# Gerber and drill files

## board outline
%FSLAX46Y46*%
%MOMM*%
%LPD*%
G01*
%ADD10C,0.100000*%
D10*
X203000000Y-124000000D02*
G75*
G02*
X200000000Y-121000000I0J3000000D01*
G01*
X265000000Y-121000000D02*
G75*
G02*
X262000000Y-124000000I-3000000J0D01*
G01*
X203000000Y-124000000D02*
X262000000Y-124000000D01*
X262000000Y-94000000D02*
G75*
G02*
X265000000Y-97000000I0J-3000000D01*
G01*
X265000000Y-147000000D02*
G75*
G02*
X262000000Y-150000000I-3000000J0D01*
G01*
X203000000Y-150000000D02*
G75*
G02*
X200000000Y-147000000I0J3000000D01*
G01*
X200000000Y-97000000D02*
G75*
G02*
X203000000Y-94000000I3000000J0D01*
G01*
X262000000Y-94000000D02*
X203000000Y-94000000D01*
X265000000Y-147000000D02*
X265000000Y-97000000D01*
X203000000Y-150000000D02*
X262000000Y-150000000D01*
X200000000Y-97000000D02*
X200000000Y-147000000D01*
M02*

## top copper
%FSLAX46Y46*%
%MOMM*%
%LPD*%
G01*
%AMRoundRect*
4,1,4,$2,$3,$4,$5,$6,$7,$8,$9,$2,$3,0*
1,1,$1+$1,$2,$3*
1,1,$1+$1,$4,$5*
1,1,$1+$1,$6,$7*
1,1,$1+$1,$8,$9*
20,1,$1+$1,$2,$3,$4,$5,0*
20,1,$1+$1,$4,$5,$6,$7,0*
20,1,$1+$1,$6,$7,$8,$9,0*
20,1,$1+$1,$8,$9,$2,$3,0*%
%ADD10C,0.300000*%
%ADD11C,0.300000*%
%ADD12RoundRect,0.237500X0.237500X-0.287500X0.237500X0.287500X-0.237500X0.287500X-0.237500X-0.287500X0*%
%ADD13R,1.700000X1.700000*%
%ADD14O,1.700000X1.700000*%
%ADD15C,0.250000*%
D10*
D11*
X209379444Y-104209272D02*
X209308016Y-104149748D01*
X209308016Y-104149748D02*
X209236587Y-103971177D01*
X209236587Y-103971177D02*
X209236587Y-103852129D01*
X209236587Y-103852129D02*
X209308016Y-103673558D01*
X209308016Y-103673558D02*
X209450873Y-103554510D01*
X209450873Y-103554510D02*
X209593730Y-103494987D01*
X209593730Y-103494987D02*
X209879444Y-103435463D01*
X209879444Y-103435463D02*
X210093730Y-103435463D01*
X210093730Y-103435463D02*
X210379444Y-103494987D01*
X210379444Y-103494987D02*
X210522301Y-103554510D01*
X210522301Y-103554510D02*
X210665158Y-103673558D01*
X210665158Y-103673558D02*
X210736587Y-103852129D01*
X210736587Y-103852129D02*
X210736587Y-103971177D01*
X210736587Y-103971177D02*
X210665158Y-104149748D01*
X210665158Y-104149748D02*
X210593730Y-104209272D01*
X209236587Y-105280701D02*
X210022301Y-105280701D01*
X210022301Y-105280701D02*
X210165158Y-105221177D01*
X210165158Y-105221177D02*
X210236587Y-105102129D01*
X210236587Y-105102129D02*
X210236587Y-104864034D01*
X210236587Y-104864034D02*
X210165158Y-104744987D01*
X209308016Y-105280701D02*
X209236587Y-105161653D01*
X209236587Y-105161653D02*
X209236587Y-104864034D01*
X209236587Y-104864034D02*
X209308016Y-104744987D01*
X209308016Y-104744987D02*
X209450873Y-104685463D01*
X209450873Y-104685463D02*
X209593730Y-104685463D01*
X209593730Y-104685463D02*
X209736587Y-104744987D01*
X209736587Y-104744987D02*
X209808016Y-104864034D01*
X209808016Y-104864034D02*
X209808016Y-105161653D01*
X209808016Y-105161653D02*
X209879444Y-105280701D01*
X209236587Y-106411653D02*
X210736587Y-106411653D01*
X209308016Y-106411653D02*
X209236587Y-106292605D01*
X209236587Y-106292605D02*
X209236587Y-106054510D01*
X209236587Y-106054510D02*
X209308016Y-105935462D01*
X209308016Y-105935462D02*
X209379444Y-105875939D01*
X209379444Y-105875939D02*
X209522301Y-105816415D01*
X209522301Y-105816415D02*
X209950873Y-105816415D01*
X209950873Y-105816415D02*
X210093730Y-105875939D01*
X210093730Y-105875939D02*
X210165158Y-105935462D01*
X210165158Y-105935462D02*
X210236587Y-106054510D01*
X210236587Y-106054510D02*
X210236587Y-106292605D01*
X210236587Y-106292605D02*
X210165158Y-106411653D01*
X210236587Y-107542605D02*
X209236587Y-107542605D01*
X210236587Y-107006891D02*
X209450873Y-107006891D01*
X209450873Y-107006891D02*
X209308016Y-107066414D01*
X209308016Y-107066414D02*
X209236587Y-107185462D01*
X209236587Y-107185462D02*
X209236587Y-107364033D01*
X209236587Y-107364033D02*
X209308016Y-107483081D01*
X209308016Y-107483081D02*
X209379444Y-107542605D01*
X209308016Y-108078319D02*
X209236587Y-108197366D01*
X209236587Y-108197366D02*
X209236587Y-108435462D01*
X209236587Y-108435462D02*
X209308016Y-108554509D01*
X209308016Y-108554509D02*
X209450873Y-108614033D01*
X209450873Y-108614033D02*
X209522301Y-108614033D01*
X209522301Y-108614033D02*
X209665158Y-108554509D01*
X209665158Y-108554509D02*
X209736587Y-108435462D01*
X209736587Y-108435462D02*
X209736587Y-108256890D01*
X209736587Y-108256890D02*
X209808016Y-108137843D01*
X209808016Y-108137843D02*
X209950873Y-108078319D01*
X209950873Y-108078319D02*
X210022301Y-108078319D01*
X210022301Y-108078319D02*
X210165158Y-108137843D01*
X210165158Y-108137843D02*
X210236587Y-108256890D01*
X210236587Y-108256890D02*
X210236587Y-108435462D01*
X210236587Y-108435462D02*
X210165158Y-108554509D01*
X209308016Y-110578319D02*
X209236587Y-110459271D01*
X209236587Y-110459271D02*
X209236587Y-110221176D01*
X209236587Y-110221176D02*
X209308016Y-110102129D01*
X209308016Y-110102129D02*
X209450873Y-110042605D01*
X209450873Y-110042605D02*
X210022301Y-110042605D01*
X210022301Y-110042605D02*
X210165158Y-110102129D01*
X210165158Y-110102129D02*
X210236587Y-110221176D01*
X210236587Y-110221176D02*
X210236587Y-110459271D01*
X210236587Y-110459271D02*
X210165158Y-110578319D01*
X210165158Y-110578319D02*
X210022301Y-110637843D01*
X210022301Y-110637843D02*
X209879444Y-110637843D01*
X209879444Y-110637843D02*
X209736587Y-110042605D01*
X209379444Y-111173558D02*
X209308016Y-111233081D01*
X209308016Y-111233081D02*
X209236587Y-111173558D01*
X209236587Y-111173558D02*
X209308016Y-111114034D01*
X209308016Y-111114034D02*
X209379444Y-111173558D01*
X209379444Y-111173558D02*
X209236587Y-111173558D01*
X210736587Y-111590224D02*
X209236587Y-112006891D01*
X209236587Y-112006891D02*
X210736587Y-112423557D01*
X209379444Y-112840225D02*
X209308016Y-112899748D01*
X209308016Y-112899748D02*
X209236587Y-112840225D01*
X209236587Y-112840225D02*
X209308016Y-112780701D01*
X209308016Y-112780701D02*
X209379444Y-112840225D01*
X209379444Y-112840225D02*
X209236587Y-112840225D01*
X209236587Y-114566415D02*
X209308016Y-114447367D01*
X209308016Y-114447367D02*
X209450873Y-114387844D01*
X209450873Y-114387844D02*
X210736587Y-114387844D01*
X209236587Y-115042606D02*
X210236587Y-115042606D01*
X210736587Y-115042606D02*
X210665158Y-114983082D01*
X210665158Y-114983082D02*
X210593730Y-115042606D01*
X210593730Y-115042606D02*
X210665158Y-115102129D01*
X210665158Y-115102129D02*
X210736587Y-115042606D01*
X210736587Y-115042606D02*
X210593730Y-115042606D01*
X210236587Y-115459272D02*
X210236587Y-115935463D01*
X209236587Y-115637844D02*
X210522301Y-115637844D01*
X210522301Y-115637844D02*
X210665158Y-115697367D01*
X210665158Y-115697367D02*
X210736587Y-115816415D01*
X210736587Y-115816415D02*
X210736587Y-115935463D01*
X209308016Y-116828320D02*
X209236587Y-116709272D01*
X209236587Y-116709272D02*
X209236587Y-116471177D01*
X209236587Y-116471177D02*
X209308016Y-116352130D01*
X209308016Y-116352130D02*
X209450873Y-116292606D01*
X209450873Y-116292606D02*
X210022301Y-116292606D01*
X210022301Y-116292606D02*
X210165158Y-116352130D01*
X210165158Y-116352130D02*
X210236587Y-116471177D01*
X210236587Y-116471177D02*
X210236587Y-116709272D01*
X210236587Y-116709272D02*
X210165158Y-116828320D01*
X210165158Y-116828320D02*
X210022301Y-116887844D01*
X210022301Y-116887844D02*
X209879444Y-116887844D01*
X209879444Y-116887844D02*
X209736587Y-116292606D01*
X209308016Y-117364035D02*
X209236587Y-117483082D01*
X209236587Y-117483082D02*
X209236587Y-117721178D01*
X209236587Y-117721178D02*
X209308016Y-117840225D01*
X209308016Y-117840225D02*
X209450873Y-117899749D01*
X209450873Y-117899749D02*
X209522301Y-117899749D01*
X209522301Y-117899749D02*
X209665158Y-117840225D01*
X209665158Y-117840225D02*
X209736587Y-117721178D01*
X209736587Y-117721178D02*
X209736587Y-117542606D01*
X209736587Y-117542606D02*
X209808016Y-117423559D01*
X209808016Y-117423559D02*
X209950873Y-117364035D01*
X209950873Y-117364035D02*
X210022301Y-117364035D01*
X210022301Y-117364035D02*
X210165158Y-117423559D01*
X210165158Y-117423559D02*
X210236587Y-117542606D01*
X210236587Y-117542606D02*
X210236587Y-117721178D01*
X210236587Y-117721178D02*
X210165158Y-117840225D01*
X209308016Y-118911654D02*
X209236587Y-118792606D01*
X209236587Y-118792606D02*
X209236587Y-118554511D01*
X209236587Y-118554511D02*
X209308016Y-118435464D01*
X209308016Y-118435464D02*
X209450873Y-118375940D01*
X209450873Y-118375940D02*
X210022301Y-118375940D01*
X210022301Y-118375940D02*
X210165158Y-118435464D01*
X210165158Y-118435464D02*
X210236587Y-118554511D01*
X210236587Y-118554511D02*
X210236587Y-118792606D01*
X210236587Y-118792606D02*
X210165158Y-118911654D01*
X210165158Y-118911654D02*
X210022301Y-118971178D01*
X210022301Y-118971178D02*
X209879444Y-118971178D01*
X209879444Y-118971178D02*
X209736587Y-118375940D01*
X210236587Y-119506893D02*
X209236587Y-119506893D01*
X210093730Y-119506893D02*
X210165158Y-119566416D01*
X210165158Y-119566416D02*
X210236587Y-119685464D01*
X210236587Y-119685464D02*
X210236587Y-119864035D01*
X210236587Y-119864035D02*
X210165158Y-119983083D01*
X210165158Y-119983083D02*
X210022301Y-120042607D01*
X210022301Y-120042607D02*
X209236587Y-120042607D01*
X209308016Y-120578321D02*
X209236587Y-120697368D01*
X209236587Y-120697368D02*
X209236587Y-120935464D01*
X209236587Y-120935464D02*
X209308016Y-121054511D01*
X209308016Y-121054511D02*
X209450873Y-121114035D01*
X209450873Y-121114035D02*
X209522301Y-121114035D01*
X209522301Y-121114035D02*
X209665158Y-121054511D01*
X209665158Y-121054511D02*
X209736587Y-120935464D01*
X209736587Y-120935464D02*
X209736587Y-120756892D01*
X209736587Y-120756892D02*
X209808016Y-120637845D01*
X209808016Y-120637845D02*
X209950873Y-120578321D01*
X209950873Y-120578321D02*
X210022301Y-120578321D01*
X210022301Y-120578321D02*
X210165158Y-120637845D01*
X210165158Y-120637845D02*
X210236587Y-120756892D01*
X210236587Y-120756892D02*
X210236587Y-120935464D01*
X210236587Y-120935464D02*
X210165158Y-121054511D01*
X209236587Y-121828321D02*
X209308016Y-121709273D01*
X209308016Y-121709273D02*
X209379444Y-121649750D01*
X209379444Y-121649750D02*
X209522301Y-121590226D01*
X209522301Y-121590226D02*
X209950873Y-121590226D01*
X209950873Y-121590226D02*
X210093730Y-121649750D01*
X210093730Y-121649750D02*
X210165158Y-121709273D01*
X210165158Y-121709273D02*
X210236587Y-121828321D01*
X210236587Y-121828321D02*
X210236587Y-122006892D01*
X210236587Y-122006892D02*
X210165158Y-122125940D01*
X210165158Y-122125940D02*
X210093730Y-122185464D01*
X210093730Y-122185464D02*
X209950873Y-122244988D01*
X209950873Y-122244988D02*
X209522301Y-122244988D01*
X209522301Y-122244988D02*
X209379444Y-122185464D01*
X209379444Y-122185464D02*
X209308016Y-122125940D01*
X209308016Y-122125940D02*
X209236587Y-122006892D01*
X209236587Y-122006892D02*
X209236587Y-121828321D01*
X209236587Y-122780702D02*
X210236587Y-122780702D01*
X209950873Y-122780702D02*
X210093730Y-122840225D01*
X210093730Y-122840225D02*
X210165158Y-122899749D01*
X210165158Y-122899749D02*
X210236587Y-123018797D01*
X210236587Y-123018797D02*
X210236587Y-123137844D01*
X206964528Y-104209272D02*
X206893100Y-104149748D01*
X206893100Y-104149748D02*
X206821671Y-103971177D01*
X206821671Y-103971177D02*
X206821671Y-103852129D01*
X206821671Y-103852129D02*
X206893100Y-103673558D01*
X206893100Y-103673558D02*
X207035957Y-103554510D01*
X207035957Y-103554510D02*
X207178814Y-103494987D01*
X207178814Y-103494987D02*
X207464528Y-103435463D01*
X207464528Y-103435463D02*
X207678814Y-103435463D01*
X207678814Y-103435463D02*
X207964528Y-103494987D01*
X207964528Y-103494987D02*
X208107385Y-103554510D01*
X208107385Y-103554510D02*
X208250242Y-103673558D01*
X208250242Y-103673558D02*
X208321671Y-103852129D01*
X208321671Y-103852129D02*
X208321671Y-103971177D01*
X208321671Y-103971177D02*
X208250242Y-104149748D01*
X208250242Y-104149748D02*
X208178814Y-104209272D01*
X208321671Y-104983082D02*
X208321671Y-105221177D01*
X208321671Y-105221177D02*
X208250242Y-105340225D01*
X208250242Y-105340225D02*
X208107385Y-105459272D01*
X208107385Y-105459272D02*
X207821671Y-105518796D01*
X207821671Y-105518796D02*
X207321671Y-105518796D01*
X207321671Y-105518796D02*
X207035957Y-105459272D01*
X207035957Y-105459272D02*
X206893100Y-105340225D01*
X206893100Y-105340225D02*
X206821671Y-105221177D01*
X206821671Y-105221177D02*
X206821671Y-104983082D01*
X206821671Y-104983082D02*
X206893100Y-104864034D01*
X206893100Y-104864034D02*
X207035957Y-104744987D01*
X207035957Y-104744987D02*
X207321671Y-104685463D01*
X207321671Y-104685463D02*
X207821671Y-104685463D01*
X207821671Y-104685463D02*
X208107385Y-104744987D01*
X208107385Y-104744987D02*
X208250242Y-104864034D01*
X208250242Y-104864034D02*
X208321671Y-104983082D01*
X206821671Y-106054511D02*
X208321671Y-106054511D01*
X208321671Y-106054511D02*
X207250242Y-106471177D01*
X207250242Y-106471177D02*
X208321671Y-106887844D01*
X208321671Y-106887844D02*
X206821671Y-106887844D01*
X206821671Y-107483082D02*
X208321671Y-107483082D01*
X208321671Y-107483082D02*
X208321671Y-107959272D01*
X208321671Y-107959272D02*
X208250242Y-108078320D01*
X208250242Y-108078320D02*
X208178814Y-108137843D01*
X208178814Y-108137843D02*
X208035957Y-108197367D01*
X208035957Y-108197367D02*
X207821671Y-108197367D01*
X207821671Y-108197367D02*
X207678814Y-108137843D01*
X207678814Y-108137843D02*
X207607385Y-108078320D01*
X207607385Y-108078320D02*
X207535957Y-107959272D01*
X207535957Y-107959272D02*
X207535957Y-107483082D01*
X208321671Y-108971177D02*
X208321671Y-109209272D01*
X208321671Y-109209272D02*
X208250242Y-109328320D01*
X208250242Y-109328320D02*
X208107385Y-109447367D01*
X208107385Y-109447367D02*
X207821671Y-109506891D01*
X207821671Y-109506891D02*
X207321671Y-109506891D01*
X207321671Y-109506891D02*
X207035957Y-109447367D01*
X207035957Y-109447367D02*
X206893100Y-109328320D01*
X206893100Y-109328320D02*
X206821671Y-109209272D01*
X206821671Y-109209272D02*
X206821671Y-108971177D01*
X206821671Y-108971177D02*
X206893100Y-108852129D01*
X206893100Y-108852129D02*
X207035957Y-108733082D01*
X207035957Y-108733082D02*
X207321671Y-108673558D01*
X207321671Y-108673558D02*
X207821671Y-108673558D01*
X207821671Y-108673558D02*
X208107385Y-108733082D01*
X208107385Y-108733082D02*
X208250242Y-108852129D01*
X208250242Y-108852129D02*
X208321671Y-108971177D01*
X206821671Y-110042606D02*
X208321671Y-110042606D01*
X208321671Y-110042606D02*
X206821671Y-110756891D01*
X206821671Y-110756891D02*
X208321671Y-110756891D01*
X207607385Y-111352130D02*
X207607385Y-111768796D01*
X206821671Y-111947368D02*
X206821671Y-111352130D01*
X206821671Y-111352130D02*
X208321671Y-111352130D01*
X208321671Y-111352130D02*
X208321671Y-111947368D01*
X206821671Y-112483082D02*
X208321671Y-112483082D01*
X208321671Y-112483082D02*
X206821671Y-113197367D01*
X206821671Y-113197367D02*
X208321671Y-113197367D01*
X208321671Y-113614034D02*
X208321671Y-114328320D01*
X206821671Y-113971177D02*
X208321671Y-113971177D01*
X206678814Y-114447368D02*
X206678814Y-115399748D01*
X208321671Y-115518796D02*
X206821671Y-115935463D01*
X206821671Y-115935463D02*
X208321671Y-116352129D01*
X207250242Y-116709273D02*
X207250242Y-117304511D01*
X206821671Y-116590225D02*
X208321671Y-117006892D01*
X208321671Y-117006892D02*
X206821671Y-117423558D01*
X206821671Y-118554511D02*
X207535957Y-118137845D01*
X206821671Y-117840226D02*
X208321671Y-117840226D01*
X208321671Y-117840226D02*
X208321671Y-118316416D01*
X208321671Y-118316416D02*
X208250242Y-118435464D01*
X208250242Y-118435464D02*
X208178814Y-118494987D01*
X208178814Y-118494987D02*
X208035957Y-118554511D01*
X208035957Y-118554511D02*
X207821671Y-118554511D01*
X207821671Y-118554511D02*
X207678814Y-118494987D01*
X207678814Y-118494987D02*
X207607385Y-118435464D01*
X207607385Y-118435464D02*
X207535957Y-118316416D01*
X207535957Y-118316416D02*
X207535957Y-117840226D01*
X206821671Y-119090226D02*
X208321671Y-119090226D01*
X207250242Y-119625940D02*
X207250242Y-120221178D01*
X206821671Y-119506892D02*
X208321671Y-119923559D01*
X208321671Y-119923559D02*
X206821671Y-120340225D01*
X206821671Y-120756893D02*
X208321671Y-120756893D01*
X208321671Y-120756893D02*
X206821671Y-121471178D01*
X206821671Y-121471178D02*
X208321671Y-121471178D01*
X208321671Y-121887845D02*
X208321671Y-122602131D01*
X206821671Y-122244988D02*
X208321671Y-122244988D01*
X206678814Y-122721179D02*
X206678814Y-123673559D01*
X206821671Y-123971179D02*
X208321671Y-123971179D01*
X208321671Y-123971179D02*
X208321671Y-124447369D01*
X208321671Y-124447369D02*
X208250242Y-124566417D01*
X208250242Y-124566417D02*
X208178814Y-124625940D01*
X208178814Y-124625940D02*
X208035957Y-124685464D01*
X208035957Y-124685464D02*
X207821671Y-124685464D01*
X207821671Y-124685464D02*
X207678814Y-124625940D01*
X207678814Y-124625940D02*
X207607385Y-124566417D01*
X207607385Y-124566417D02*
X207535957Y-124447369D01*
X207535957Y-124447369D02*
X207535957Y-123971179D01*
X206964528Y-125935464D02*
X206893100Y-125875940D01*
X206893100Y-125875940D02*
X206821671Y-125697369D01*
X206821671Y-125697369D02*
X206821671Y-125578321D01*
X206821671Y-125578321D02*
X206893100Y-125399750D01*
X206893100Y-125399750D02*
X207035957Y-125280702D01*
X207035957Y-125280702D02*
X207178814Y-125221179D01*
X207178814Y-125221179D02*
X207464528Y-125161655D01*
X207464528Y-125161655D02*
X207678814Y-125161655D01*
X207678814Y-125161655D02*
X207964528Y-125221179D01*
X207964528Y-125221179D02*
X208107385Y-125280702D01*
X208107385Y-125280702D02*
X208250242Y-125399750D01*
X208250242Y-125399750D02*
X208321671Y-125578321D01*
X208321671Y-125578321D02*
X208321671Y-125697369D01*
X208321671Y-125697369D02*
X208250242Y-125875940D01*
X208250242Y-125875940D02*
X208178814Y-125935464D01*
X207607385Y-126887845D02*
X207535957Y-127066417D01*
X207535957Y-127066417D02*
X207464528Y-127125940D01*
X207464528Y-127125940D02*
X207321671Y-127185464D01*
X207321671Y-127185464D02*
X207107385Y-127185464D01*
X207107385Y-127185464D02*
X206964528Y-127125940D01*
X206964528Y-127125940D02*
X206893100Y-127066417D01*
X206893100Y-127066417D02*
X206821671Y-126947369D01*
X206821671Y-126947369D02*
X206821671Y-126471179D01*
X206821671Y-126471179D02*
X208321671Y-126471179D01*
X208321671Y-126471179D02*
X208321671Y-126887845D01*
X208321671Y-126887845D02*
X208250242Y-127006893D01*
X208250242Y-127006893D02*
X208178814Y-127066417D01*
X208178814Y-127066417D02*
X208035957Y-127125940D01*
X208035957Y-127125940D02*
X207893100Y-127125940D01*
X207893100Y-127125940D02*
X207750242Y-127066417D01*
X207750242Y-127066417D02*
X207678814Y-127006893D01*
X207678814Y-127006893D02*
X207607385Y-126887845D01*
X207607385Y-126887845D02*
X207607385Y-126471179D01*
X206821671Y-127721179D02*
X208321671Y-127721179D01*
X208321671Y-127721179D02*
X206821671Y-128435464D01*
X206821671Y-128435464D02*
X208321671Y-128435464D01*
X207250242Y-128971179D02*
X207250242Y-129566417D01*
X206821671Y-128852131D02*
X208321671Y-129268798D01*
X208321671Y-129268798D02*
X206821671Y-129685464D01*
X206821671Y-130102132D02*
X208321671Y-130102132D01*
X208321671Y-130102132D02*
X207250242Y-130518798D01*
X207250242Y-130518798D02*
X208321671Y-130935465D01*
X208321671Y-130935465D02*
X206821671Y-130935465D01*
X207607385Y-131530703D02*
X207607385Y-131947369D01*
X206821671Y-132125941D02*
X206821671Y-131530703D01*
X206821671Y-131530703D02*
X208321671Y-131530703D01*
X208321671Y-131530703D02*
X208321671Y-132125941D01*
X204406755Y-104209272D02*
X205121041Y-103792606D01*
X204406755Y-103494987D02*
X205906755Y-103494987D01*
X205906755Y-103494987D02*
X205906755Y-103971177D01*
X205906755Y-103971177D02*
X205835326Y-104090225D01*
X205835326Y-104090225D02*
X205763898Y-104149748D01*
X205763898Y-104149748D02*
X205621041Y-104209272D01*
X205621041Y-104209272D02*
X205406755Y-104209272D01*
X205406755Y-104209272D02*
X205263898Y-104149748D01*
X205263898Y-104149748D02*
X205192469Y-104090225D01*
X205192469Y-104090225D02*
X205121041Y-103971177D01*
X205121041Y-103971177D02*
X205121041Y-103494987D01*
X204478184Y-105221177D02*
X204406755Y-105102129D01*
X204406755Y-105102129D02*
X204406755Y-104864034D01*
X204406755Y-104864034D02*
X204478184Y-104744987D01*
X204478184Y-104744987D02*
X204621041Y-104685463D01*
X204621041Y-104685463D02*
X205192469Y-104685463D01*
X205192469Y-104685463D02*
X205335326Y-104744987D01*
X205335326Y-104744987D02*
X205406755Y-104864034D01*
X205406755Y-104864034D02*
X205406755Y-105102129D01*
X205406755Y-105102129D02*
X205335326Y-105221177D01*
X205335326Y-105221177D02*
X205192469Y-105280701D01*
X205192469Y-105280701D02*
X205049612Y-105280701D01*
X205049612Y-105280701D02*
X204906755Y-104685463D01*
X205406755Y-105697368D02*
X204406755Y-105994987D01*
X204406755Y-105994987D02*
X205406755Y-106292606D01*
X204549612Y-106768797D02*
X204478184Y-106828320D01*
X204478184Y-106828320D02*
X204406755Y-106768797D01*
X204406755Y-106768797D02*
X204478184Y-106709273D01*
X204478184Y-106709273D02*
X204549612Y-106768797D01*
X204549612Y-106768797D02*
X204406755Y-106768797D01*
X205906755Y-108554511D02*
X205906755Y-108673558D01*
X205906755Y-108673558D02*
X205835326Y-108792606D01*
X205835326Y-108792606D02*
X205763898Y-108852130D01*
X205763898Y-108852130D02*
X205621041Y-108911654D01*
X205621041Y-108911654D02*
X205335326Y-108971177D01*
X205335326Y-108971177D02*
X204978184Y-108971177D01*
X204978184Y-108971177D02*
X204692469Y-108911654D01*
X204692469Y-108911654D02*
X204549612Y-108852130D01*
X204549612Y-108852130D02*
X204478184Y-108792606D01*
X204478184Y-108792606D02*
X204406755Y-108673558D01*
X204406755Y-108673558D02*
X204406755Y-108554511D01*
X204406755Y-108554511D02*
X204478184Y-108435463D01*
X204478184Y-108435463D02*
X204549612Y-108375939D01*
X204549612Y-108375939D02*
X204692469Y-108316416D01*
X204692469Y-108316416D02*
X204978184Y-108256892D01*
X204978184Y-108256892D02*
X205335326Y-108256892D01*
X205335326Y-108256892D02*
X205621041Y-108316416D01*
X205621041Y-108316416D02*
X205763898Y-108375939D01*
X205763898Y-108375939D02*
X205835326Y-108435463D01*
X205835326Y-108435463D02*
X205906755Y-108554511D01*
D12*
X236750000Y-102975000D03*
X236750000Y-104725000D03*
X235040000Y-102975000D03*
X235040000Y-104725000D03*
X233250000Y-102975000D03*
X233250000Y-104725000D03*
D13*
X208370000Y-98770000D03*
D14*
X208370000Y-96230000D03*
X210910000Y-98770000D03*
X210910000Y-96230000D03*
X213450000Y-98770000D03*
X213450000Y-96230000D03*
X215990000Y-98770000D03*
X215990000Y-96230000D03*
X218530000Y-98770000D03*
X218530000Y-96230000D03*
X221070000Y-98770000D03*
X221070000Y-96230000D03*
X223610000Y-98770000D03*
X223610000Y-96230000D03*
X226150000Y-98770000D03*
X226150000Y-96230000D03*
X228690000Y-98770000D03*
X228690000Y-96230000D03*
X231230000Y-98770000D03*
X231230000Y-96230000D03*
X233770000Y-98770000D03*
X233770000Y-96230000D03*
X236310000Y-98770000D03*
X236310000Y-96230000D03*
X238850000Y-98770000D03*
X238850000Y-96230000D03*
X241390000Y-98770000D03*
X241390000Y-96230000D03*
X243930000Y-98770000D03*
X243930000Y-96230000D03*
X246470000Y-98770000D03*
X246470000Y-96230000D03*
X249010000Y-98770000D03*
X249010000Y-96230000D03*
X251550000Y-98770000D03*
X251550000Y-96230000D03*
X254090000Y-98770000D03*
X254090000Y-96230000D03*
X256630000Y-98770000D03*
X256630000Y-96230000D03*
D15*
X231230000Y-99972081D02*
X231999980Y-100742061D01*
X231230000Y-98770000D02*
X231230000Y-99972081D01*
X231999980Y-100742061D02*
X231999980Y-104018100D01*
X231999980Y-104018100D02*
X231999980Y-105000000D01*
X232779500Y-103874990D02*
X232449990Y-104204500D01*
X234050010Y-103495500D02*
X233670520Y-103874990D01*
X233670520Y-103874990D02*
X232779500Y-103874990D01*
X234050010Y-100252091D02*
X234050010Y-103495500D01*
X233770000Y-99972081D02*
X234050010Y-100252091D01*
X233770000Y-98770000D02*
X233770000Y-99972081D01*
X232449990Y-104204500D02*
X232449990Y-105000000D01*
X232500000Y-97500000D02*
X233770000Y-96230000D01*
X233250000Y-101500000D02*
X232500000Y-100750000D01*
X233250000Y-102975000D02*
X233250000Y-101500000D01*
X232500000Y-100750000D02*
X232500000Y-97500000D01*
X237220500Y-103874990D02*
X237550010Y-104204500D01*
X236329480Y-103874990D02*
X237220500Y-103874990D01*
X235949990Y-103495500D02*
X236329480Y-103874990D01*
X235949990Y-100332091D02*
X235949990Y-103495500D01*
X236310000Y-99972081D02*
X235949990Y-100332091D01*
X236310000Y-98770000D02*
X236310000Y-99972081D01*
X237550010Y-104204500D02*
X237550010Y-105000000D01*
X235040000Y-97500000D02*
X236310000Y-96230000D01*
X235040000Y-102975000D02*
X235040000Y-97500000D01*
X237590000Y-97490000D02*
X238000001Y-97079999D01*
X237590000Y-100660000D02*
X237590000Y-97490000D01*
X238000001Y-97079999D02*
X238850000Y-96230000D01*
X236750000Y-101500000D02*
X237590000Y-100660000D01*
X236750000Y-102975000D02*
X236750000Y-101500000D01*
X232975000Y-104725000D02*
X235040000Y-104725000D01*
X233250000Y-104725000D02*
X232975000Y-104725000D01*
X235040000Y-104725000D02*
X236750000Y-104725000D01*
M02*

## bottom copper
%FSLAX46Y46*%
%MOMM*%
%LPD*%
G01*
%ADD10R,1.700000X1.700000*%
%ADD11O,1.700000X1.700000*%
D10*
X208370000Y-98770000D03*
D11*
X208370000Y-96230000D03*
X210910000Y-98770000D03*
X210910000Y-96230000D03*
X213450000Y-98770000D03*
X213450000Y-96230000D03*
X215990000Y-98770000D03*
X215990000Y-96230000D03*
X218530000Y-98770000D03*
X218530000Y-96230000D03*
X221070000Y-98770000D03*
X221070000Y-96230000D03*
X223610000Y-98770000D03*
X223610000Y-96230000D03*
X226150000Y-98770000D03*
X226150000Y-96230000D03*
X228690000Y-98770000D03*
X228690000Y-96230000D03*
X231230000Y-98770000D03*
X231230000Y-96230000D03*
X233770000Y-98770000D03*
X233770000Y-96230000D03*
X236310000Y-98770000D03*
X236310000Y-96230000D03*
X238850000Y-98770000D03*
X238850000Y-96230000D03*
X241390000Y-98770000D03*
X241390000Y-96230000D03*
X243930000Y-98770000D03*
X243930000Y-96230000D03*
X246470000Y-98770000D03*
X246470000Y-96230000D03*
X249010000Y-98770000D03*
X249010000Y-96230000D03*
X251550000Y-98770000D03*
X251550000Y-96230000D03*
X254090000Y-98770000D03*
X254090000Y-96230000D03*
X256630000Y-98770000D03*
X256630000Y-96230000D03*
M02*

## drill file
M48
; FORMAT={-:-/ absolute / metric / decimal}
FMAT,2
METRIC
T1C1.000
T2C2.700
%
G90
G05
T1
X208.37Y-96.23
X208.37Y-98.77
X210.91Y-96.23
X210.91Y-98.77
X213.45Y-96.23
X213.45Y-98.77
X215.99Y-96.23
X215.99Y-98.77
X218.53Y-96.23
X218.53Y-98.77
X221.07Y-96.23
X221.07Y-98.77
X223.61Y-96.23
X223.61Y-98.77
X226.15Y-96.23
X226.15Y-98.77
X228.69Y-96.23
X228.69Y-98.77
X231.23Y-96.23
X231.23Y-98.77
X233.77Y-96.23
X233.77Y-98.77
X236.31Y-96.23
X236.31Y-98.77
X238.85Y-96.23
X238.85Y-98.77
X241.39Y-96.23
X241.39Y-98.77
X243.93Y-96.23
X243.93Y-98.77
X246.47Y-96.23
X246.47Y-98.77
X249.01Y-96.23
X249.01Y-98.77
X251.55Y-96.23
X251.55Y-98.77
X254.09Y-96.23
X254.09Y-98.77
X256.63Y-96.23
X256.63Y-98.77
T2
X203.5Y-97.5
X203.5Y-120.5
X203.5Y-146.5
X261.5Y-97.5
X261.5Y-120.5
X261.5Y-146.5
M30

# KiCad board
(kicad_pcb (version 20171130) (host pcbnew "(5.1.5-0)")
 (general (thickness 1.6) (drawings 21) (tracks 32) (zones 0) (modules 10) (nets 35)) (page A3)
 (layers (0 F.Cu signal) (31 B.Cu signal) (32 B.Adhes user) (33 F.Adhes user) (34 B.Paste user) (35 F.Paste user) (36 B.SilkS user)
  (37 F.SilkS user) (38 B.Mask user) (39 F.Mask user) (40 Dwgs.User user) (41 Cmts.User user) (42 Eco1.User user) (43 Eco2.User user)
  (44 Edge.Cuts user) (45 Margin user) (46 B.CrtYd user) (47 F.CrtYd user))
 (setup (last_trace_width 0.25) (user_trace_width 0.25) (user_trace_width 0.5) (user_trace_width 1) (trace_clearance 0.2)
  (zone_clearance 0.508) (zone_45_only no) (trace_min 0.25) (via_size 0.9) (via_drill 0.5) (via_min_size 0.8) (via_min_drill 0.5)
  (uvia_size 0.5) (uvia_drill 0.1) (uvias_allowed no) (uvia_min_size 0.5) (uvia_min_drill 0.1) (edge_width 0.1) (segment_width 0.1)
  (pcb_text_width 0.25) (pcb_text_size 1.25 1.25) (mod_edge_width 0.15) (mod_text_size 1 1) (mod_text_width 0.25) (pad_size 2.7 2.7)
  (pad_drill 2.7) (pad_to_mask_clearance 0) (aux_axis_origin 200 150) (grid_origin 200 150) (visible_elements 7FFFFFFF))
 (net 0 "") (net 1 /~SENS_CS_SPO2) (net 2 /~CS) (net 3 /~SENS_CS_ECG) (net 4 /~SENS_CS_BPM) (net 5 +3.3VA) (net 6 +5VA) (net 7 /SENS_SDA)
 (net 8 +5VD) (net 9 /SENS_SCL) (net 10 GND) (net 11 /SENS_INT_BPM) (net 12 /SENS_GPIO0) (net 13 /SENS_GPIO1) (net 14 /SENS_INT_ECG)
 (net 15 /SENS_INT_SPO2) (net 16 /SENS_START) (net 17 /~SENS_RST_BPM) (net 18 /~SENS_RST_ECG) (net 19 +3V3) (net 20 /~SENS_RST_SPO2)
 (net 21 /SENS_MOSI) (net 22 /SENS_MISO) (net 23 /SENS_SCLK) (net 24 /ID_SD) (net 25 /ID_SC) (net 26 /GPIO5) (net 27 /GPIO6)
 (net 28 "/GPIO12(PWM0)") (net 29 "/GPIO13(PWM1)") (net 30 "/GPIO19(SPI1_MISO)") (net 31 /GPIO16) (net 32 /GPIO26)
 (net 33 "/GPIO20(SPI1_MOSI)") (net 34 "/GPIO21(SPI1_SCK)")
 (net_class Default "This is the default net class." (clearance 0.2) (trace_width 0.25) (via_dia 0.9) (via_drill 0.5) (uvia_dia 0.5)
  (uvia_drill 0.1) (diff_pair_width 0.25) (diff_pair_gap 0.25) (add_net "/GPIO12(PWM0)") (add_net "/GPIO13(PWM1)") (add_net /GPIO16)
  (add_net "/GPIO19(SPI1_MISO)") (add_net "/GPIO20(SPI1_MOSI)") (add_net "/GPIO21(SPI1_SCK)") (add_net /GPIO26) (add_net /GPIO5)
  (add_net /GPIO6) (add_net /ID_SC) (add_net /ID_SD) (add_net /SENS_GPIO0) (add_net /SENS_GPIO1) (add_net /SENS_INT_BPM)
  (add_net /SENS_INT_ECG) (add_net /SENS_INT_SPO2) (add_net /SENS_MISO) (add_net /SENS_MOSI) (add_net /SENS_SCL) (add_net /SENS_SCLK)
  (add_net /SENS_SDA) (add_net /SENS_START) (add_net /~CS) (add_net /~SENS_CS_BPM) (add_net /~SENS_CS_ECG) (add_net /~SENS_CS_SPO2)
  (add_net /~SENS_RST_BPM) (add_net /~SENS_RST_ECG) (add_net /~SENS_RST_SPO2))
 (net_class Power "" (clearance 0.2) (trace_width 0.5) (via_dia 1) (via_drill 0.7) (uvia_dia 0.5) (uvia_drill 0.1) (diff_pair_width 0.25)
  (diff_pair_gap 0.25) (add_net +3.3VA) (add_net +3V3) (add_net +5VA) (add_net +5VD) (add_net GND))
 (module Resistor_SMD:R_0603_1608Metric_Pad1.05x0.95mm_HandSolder (layer F.Cu) (at 236.75 103.85 90)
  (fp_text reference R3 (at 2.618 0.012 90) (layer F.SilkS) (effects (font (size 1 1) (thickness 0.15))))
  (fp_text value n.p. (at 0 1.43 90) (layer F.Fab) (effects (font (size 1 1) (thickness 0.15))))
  (pad 2 smd roundrect (at 0.875 0 90) (size 1.05 0.95) (layers F.Cu F.Paste F.Mask) (roundrect_rratio 0.25) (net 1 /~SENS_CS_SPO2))
  (pad 1 smd roundrect (at -0.875 0 90) (size 1.05 0.95) (layers F.Cu F.Paste F.Mask) (roundrect_rratio 0.25) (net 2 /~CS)))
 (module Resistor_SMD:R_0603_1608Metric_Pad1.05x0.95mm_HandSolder (layer F.Cu) (at 235.04 103.85 90)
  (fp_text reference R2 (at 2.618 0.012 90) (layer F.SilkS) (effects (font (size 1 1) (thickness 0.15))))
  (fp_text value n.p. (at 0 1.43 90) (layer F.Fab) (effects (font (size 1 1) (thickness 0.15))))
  (pad 2 smd roundrect (at 0.875 0 90) (size 1.05 0.95) (layers F.Cu F.Paste F.Mask) (roundrect_rratio 0.25) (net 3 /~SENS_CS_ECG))
  (pad 1 smd roundrect (at -0.875 0 90) (size 1.05 0.95) (layers F.Cu F.Paste F.Mask) (roundrect_rratio 0.25) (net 2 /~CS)))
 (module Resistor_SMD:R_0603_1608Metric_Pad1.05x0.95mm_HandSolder (layer F.Cu) (at 233.25 103.85 90)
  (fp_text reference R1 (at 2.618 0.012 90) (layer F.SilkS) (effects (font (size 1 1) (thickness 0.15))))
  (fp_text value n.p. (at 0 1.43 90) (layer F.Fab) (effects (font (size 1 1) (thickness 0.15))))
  (pad 2 smd roundrect (at 0.875 0 90) (size 1.05 0.95) (layers F.Cu F.Paste F.Mask) (roundrect_rratio 0.25) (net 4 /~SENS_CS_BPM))
  (pad 1 smd roundrect (at -0.875 0 90) (size 1.05 0.95) (layers F.Cu F.Paste F.Mask) (roundrect_rratio 0.25) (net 2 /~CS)))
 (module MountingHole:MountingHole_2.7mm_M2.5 (layer F.Cu) (at 261.5 146.5)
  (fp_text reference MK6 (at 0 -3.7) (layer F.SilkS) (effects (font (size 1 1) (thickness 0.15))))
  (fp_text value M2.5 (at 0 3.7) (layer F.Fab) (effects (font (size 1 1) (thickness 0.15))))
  (pad 1 np_thru_hole circle (at 0 0) (size 2.7 2.7) (drill 2.7) (layers *.Cu *.Mask)))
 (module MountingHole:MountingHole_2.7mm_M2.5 (layer F.Cu) (at 203.5 146.5)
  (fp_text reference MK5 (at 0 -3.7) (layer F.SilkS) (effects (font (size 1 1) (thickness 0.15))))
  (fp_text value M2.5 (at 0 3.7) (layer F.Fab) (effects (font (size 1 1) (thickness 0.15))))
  (pad 1 np_thru_hole circle (at 0 0) (size 2.7 2.7) (drill 2.7) (layers *.Cu *.Mask)))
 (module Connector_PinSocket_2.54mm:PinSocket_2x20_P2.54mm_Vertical (layer B.Cu) (at 208.37 98.77 270)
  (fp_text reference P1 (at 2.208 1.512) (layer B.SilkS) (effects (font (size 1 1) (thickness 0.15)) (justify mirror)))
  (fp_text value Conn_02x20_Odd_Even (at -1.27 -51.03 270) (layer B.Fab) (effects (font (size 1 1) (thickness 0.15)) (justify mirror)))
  (pad 1 thru_hole rect (at 0 0 270) (size 1.7 1.7) (drill 1) (layers *.Cu *.Mask) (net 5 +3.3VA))
  (pad 2 thru_hole oval (at -2.54 0 270) (size 1.7 1.7) (drill 1) (layers *.Cu *.Mask) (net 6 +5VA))
  (pad 3 thru_hole oval (at 0 -2.54 270) (size 1.7 1.7) (drill 1) (layers *.Cu *.Mask) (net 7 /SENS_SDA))
  (pad 4 thru_hole oval (at -2.54 -2.54 270) (size 1.7 1.7) (drill 1) (layers *.Cu *.Mask) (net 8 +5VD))
  (pad 5 thru_hole oval (at 0 -5.08 270) (size 1.7 1.7) (drill 1) (layers *.Cu *.Mask) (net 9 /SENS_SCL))
  (pad 6 thru_hole oval (at -2.54 -5.08 270) (size 1.7 1.7) (drill 1) (layers *.Cu *.Mask) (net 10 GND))
  (pad 7 thru_hole oval (at 0 -7.62 270) (size 1.7 1.7) (drill 1) (layers *.Cu *.Mask) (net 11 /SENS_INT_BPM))
  (pad 8 thru_hole oval (at -2.54 -7.62 270) (size 1.7 1.7) (drill 1) (layers *.Cu *.Mask) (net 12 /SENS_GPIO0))
  (pad 9 thru_hole oval (at 0 -10.16 270) (size 1.7 1.7) (drill 1) (layers *.Cu *.Mask) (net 10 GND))
  (pad 10 thru_hole oval (at -2.54 -10.16 270) (size 1.7 1.7) (drill 1) (layers *.Cu *.Mask) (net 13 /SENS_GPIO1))
  (pad 11 thru_hole oval (at 0 -12.7 270) (size 1.7 1.7) (drill 1) (layers *.Cu *.Mask) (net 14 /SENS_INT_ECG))
  (pad 12 thru_hole oval (at -2.54 -12.7 270) (size 1.7 1.7) (drill 1) (layers *.Cu *.Mask) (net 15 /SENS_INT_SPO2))
  (pad 13 thru_hole oval (at 0 -15.24 270) (size 1.7 1.7) (drill 1) (layers *.Cu *.Mask) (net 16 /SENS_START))
  (pad 14 thru_hole oval (at -2.54 -15.24 270) (size 1.7 1.7) (drill 1) (layers *.Cu *.Mask) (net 10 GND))
  (pad 15 thru_hole oval (at 0 -17.78 270) (size 1.7 1.7) (drill 1) (layers *.Cu *.Mask) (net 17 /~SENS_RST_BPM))
  (pad 16 thru_hole oval (at -2.54 -17.78 270) (size 1.7 1.7) (drill 1) (layers *.Cu *.Mask) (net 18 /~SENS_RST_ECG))
  (pad 17 thru_hole oval (at 0 -20.32 270) (size 1.7 1.7) (drill 1) (layers *.Cu *.Mask) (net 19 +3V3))
  (pad 18 thru_hole oval (at -2.54 -20.32 270) (size 1.7 1.7) (drill 1) (layers *.Cu *.Mask) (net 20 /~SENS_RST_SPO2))
  (pad 19 thru_hole oval (at 0 -22.86 270) (size 1.7 1.7) (drill 1) (layers *.Cu *.Mask) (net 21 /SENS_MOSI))
  (pad 20 thru_hole oval (at -2.54 -22.86 270) (size 1.7 1.7) (drill 1) (layers *.Cu *.Mask) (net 10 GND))
  (pad 21 thru_hole oval (at 0 -25.4 270) (size 1.7 1.7) (drill 1) (layers *.Cu *.Mask) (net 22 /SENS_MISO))
  (pad 22 thru_hole oval (at -2.54 -25.4 270) (size 1.7 1.7) (drill 1) (layers *.Cu *.Mask) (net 4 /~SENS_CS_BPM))
  (pad 23 thru_hole oval (at 0 -27.94 270) (size 1.7 1.7) (drill 1) (layers *.Cu *.Mask) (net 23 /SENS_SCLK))
  (pad 24 thru_hole oval (at -2.54 -27.94 270) (size 1.7 1.7) (drill 1) (layers *.Cu *.Mask) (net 3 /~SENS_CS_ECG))
  (pad 25 thru_hole oval (at 0 -30.48 270) (size 1.7 1.7) (drill 1) (layers *.Cu *.Mask) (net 10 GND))
  (pad 26 thru_hole oval (at -2.54 -30.48 270) (size 1.7 1.7) (drill 1) (layers *.Cu *.Mask) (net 1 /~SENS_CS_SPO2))
  (pad 27 thru_hole oval (at 0 -33.02 270) (size 1.7 1.7) (drill 1) (layers *.Cu *.Mask) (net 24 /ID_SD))
  (pad 28 thru_hole oval (at -2.54 -33.02 270) (size 1.7 1.7) (drill 1) (layers *.Cu *.Mask) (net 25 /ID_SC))
  (pad 29 thru_hole oval (at 0 -35.56 270) (size 1.7 1.7) (drill 1) (layers *.Cu *.Mask) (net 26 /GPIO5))
  (pad 30 thru_hole oval (at -2.54 -35.56 270) (size 1.7 1.7) (drill 1) (layers *.Cu *.Mask) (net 10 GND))
  (pad 31 thru_hole oval (at 0 -38.1 270) (size 1.7 1.7) (drill 1) (layers *.Cu *.Mask) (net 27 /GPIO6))
  (pad 32 thru_hole oval (at -2.54 -38.1 270) (size 1.7 1.7) (drill 1) (layers *.Cu *.Mask) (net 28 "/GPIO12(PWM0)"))
  (pad 33 thru_hole oval (at 0 -40.64 270) (size 1.7 1.7) (drill 1) (layers *.Cu *.Mask) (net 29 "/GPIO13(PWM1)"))
  (pad 34 thru_hole oval (at -2.54 -40.64 270) (size 1.7 1.7) (drill 1) (layers *.Cu *.Mask) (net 10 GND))
  (pad 35 thru_hole oval (at 0 -43.18 270) (size 1.7 1.7) (drill 1) (layers *.Cu *.Mask) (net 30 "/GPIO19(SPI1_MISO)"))
  (pad 36 thru_hole oval (at -2.54 -43.18 270) (size 1.7 1.7) (drill 1) (layers *.Cu *.Mask) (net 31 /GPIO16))
  (pad 37 thru_hole oval (at 0 -45.72 270) (size 1.7 1.7) (drill 1) (layers *.Cu *.Mask) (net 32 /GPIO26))
  (pad 38 thru_hole oval (at -2.54 -45.72 270) (size 1.7 1.7) (drill 1) (layers *.Cu *.Mask) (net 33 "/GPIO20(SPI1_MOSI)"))
  (pad 39 thru_hole oval (at 0 -48.26 270) (size 1.7 1.7) (drill 1) (layers *.Cu *.Mask) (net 10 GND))
  (pad 40 thru_hole oval (at -2.54 -48.26 270) (size 1.7 1.7) (drill 1) (layers *.Cu *.Mask) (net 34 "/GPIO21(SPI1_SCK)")))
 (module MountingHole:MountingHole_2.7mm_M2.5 (layer F.Cu) (at 261.5 120.5)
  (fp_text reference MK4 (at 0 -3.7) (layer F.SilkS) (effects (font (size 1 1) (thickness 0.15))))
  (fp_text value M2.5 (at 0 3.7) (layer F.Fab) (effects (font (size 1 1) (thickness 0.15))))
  (pad 1 np_thru_hole circle (at 0 0) (size 2.7 2.7) (drill 2.7) (layers *.Cu *.Mask)))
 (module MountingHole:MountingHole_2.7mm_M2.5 (layer F.Cu) (at 203.5 120.5)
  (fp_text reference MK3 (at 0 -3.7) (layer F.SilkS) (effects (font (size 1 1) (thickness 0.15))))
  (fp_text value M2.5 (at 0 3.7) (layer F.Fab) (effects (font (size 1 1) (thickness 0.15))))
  (pad 1 np_thru_hole circle (at 0 0) (size 2.7 2.7) (drill 2.7) (layers *.Cu *.Mask)))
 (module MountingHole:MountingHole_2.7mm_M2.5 (layer F.Cu) (at 261.5 97.5 180)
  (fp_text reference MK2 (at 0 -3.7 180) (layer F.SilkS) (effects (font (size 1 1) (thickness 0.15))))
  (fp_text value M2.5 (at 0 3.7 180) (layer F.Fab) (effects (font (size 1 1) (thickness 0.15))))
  (pad 1 np_thru_hole circle (at 0 0 180) (size 2.7 2.7) (drill 2.7) (layers *.Cu *.Mask)))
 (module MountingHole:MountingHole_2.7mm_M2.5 (layer F.Cu) (at 203.5 97.5 180)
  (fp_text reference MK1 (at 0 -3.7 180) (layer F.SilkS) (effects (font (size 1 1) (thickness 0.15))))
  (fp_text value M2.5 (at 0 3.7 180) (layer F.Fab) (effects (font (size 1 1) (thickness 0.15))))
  (pad 1 np_thru_hole circle (at 0 0 180) (size 2.7 2.7) (drill 2.7) (layers *.Cu *.Mask)))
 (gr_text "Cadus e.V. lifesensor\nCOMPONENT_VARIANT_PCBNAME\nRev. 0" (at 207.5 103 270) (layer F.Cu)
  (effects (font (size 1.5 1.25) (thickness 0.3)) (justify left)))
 (gr_arc (start 203 121) (end 200 121) (angle -90) (layer Edge.Cuts) (width 0.1))
 (gr_arc (start 262 121) (end 262 124) (angle -90) (layer Edge.Cuts) (width 0.1))
 (gr_line (start 203 124) (end 262 124) (layer Edge.Cuts) (width 0.1))
 (gr_arc (start 262 97) (end 262 94) (angle 90) (layer Edge.Cuts) (width 0.1))
 (gr_arc (start 262 147) (end 265 147) (angle 90) (layer Edge.Cuts) (width 0.1))
 (gr_arc (start 203 147) (end 203 150) (angle 90) (layer Edge.Cuts) (width 0.1))
 (gr_arc (start 203 97) (end 200 97) (angle 90) (layer Edge.Cuts) (width 0.1))
 (gr_line (start 262 94) (end 203 94) (layer Edge.Cuts) (width 0.1))
 (gr_line (start 265 147) (end 265 97) (layer Edge.Cuts) (width 0.1))
 (gr_line (start 203 150) (end 262 150) (layer Edge.Cuts) (width 0.1))
 (gr_line (start 200 97) (end 200 147) (layer Edge.Cuts) (width 0.1))
 (segment (start 231.23 99.972081) (end 231.99998 100.742061) (width 0.25) (layer F.Cu) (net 21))
 (segment (start 231.23 98.77) (end 231.23 99.972081) (width 0.25) (layer F.Cu) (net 21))
 (segment (start 231.99998 100.742061) (end 231.99998 104.0181) (width 0.25) (layer F.Cu) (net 21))
 (segment (start 231.99998 104.0181) (end 231.99998 105) (width 0.25) (layer F.Cu) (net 21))
 (segment (start 232.7795 103.87499) (end 232.44999 104.2045) (width 0.25) (layer F.Cu) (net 22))
 (segment (start 234.05001 103.4955) (end 233.67052 103.87499) (width 0.25) (layer F.Cu) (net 22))
 (segment (start 233.67052 103.87499) (end 232.7795 103.87499) (width 0.25) (layer F.Cu) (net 22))
 (segment (start 234.05001 100.252091) (end 234.05001 103.4955) (width 0.25) (layer F.Cu) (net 22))
 (segment (start 233.77 99.972081) (end 234.05001 100.252091) (width 0.25) (layer F.Cu) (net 22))
 (segment (start 233.77 98.77) (end 233.77 99.972081) (width 0.25) (layer F.Cu) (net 22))
 (segment (start 232.44999 104.2045) (end 232.44999 105) (width 0.25) (layer F.Cu) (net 22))
 (segment (start 232.5 97.5) (end 233.77 96.23) (width 0.25) (layer F.Cu) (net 4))
 (segment (start 233.25 101.5) (end 232.5 100.75) (width 0.25) (layer F.Cu) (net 4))
 (segment (start 233.25 102.975) (end 233.25 101.5) (width 0.25) (layer F.Cu) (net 4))
 (segment (start 232.5 100.75) (end 232.5 97.5) (width 0.25) (layer F.Cu) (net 4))
 (segment (start 237.2205 103.87499) (end 237.55001 104.2045) (width 0.25) (layer F.Cu) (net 23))
 (segment (start 236.32948 103.87499) (end 237.2205 103.87499) (width 0.25) (layer F.Cu) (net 23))
 (segment (start 235.94999 103.4955) (end 236.32948 103.87499) (width 0.25) (layer F.Cu) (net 23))
 (segment (start 235.94999 100.332091) (end 235.94999 103.4955) (width 0.25) (layer F.Cu) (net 23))
 (segment (start 236.31 99.972081) (end 235.94999 100.332091) (width 0.25) (layer F.Cu) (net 23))
 (segment (start 236.31 98.77) (end 236.31 99.972081) (width 0.25) (layer F.Cu) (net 23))
 (segment (start 237.55001 104.2045) (end 237.55001 105) (width 0.25) (layer F.Cu) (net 23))
 (segment (start 235.04 97.5) (end 236.31 96.23) (width 0.25) (layer F.Cu) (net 3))
 (segment (start 235.04 102.975) (end 235.04 97.5) (width 0.25) (layer F.Cu) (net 3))
 (segment (start 237.59 97.49) (end 238.000001 97.079999) (width 0.25) (layer F.Cu) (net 1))
 (segment (start 237.59 100.66) (end 237.59 97.49) (width 0.25) (layer F.Cu) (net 1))
 (segment (start 238.000001 97.079999) (end 238.85 96.23) (width 0.25) (layer F.Cu) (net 1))
 (segment (start 236.75 101.5) (end 237.59 100.66) (width 0.25) (layer F.Cu) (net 1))
 (segment (start 236.75 102.975) (end 236.75 101.5) (width 0.25) (layer F.Cu) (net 1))
 (segment (start 232.975 104.725) (end 235.04 104.725) (width 0.25) (layer F.Cu) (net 2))
 (segment (start 233.25 104.725) (end 232.975 104.725) (width 0.25) (layer F.Cu) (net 2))
 (segment (start 235.04 104.725) (end 236.75 104.725) (width 0.25) (layer F.Cu) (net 2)))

